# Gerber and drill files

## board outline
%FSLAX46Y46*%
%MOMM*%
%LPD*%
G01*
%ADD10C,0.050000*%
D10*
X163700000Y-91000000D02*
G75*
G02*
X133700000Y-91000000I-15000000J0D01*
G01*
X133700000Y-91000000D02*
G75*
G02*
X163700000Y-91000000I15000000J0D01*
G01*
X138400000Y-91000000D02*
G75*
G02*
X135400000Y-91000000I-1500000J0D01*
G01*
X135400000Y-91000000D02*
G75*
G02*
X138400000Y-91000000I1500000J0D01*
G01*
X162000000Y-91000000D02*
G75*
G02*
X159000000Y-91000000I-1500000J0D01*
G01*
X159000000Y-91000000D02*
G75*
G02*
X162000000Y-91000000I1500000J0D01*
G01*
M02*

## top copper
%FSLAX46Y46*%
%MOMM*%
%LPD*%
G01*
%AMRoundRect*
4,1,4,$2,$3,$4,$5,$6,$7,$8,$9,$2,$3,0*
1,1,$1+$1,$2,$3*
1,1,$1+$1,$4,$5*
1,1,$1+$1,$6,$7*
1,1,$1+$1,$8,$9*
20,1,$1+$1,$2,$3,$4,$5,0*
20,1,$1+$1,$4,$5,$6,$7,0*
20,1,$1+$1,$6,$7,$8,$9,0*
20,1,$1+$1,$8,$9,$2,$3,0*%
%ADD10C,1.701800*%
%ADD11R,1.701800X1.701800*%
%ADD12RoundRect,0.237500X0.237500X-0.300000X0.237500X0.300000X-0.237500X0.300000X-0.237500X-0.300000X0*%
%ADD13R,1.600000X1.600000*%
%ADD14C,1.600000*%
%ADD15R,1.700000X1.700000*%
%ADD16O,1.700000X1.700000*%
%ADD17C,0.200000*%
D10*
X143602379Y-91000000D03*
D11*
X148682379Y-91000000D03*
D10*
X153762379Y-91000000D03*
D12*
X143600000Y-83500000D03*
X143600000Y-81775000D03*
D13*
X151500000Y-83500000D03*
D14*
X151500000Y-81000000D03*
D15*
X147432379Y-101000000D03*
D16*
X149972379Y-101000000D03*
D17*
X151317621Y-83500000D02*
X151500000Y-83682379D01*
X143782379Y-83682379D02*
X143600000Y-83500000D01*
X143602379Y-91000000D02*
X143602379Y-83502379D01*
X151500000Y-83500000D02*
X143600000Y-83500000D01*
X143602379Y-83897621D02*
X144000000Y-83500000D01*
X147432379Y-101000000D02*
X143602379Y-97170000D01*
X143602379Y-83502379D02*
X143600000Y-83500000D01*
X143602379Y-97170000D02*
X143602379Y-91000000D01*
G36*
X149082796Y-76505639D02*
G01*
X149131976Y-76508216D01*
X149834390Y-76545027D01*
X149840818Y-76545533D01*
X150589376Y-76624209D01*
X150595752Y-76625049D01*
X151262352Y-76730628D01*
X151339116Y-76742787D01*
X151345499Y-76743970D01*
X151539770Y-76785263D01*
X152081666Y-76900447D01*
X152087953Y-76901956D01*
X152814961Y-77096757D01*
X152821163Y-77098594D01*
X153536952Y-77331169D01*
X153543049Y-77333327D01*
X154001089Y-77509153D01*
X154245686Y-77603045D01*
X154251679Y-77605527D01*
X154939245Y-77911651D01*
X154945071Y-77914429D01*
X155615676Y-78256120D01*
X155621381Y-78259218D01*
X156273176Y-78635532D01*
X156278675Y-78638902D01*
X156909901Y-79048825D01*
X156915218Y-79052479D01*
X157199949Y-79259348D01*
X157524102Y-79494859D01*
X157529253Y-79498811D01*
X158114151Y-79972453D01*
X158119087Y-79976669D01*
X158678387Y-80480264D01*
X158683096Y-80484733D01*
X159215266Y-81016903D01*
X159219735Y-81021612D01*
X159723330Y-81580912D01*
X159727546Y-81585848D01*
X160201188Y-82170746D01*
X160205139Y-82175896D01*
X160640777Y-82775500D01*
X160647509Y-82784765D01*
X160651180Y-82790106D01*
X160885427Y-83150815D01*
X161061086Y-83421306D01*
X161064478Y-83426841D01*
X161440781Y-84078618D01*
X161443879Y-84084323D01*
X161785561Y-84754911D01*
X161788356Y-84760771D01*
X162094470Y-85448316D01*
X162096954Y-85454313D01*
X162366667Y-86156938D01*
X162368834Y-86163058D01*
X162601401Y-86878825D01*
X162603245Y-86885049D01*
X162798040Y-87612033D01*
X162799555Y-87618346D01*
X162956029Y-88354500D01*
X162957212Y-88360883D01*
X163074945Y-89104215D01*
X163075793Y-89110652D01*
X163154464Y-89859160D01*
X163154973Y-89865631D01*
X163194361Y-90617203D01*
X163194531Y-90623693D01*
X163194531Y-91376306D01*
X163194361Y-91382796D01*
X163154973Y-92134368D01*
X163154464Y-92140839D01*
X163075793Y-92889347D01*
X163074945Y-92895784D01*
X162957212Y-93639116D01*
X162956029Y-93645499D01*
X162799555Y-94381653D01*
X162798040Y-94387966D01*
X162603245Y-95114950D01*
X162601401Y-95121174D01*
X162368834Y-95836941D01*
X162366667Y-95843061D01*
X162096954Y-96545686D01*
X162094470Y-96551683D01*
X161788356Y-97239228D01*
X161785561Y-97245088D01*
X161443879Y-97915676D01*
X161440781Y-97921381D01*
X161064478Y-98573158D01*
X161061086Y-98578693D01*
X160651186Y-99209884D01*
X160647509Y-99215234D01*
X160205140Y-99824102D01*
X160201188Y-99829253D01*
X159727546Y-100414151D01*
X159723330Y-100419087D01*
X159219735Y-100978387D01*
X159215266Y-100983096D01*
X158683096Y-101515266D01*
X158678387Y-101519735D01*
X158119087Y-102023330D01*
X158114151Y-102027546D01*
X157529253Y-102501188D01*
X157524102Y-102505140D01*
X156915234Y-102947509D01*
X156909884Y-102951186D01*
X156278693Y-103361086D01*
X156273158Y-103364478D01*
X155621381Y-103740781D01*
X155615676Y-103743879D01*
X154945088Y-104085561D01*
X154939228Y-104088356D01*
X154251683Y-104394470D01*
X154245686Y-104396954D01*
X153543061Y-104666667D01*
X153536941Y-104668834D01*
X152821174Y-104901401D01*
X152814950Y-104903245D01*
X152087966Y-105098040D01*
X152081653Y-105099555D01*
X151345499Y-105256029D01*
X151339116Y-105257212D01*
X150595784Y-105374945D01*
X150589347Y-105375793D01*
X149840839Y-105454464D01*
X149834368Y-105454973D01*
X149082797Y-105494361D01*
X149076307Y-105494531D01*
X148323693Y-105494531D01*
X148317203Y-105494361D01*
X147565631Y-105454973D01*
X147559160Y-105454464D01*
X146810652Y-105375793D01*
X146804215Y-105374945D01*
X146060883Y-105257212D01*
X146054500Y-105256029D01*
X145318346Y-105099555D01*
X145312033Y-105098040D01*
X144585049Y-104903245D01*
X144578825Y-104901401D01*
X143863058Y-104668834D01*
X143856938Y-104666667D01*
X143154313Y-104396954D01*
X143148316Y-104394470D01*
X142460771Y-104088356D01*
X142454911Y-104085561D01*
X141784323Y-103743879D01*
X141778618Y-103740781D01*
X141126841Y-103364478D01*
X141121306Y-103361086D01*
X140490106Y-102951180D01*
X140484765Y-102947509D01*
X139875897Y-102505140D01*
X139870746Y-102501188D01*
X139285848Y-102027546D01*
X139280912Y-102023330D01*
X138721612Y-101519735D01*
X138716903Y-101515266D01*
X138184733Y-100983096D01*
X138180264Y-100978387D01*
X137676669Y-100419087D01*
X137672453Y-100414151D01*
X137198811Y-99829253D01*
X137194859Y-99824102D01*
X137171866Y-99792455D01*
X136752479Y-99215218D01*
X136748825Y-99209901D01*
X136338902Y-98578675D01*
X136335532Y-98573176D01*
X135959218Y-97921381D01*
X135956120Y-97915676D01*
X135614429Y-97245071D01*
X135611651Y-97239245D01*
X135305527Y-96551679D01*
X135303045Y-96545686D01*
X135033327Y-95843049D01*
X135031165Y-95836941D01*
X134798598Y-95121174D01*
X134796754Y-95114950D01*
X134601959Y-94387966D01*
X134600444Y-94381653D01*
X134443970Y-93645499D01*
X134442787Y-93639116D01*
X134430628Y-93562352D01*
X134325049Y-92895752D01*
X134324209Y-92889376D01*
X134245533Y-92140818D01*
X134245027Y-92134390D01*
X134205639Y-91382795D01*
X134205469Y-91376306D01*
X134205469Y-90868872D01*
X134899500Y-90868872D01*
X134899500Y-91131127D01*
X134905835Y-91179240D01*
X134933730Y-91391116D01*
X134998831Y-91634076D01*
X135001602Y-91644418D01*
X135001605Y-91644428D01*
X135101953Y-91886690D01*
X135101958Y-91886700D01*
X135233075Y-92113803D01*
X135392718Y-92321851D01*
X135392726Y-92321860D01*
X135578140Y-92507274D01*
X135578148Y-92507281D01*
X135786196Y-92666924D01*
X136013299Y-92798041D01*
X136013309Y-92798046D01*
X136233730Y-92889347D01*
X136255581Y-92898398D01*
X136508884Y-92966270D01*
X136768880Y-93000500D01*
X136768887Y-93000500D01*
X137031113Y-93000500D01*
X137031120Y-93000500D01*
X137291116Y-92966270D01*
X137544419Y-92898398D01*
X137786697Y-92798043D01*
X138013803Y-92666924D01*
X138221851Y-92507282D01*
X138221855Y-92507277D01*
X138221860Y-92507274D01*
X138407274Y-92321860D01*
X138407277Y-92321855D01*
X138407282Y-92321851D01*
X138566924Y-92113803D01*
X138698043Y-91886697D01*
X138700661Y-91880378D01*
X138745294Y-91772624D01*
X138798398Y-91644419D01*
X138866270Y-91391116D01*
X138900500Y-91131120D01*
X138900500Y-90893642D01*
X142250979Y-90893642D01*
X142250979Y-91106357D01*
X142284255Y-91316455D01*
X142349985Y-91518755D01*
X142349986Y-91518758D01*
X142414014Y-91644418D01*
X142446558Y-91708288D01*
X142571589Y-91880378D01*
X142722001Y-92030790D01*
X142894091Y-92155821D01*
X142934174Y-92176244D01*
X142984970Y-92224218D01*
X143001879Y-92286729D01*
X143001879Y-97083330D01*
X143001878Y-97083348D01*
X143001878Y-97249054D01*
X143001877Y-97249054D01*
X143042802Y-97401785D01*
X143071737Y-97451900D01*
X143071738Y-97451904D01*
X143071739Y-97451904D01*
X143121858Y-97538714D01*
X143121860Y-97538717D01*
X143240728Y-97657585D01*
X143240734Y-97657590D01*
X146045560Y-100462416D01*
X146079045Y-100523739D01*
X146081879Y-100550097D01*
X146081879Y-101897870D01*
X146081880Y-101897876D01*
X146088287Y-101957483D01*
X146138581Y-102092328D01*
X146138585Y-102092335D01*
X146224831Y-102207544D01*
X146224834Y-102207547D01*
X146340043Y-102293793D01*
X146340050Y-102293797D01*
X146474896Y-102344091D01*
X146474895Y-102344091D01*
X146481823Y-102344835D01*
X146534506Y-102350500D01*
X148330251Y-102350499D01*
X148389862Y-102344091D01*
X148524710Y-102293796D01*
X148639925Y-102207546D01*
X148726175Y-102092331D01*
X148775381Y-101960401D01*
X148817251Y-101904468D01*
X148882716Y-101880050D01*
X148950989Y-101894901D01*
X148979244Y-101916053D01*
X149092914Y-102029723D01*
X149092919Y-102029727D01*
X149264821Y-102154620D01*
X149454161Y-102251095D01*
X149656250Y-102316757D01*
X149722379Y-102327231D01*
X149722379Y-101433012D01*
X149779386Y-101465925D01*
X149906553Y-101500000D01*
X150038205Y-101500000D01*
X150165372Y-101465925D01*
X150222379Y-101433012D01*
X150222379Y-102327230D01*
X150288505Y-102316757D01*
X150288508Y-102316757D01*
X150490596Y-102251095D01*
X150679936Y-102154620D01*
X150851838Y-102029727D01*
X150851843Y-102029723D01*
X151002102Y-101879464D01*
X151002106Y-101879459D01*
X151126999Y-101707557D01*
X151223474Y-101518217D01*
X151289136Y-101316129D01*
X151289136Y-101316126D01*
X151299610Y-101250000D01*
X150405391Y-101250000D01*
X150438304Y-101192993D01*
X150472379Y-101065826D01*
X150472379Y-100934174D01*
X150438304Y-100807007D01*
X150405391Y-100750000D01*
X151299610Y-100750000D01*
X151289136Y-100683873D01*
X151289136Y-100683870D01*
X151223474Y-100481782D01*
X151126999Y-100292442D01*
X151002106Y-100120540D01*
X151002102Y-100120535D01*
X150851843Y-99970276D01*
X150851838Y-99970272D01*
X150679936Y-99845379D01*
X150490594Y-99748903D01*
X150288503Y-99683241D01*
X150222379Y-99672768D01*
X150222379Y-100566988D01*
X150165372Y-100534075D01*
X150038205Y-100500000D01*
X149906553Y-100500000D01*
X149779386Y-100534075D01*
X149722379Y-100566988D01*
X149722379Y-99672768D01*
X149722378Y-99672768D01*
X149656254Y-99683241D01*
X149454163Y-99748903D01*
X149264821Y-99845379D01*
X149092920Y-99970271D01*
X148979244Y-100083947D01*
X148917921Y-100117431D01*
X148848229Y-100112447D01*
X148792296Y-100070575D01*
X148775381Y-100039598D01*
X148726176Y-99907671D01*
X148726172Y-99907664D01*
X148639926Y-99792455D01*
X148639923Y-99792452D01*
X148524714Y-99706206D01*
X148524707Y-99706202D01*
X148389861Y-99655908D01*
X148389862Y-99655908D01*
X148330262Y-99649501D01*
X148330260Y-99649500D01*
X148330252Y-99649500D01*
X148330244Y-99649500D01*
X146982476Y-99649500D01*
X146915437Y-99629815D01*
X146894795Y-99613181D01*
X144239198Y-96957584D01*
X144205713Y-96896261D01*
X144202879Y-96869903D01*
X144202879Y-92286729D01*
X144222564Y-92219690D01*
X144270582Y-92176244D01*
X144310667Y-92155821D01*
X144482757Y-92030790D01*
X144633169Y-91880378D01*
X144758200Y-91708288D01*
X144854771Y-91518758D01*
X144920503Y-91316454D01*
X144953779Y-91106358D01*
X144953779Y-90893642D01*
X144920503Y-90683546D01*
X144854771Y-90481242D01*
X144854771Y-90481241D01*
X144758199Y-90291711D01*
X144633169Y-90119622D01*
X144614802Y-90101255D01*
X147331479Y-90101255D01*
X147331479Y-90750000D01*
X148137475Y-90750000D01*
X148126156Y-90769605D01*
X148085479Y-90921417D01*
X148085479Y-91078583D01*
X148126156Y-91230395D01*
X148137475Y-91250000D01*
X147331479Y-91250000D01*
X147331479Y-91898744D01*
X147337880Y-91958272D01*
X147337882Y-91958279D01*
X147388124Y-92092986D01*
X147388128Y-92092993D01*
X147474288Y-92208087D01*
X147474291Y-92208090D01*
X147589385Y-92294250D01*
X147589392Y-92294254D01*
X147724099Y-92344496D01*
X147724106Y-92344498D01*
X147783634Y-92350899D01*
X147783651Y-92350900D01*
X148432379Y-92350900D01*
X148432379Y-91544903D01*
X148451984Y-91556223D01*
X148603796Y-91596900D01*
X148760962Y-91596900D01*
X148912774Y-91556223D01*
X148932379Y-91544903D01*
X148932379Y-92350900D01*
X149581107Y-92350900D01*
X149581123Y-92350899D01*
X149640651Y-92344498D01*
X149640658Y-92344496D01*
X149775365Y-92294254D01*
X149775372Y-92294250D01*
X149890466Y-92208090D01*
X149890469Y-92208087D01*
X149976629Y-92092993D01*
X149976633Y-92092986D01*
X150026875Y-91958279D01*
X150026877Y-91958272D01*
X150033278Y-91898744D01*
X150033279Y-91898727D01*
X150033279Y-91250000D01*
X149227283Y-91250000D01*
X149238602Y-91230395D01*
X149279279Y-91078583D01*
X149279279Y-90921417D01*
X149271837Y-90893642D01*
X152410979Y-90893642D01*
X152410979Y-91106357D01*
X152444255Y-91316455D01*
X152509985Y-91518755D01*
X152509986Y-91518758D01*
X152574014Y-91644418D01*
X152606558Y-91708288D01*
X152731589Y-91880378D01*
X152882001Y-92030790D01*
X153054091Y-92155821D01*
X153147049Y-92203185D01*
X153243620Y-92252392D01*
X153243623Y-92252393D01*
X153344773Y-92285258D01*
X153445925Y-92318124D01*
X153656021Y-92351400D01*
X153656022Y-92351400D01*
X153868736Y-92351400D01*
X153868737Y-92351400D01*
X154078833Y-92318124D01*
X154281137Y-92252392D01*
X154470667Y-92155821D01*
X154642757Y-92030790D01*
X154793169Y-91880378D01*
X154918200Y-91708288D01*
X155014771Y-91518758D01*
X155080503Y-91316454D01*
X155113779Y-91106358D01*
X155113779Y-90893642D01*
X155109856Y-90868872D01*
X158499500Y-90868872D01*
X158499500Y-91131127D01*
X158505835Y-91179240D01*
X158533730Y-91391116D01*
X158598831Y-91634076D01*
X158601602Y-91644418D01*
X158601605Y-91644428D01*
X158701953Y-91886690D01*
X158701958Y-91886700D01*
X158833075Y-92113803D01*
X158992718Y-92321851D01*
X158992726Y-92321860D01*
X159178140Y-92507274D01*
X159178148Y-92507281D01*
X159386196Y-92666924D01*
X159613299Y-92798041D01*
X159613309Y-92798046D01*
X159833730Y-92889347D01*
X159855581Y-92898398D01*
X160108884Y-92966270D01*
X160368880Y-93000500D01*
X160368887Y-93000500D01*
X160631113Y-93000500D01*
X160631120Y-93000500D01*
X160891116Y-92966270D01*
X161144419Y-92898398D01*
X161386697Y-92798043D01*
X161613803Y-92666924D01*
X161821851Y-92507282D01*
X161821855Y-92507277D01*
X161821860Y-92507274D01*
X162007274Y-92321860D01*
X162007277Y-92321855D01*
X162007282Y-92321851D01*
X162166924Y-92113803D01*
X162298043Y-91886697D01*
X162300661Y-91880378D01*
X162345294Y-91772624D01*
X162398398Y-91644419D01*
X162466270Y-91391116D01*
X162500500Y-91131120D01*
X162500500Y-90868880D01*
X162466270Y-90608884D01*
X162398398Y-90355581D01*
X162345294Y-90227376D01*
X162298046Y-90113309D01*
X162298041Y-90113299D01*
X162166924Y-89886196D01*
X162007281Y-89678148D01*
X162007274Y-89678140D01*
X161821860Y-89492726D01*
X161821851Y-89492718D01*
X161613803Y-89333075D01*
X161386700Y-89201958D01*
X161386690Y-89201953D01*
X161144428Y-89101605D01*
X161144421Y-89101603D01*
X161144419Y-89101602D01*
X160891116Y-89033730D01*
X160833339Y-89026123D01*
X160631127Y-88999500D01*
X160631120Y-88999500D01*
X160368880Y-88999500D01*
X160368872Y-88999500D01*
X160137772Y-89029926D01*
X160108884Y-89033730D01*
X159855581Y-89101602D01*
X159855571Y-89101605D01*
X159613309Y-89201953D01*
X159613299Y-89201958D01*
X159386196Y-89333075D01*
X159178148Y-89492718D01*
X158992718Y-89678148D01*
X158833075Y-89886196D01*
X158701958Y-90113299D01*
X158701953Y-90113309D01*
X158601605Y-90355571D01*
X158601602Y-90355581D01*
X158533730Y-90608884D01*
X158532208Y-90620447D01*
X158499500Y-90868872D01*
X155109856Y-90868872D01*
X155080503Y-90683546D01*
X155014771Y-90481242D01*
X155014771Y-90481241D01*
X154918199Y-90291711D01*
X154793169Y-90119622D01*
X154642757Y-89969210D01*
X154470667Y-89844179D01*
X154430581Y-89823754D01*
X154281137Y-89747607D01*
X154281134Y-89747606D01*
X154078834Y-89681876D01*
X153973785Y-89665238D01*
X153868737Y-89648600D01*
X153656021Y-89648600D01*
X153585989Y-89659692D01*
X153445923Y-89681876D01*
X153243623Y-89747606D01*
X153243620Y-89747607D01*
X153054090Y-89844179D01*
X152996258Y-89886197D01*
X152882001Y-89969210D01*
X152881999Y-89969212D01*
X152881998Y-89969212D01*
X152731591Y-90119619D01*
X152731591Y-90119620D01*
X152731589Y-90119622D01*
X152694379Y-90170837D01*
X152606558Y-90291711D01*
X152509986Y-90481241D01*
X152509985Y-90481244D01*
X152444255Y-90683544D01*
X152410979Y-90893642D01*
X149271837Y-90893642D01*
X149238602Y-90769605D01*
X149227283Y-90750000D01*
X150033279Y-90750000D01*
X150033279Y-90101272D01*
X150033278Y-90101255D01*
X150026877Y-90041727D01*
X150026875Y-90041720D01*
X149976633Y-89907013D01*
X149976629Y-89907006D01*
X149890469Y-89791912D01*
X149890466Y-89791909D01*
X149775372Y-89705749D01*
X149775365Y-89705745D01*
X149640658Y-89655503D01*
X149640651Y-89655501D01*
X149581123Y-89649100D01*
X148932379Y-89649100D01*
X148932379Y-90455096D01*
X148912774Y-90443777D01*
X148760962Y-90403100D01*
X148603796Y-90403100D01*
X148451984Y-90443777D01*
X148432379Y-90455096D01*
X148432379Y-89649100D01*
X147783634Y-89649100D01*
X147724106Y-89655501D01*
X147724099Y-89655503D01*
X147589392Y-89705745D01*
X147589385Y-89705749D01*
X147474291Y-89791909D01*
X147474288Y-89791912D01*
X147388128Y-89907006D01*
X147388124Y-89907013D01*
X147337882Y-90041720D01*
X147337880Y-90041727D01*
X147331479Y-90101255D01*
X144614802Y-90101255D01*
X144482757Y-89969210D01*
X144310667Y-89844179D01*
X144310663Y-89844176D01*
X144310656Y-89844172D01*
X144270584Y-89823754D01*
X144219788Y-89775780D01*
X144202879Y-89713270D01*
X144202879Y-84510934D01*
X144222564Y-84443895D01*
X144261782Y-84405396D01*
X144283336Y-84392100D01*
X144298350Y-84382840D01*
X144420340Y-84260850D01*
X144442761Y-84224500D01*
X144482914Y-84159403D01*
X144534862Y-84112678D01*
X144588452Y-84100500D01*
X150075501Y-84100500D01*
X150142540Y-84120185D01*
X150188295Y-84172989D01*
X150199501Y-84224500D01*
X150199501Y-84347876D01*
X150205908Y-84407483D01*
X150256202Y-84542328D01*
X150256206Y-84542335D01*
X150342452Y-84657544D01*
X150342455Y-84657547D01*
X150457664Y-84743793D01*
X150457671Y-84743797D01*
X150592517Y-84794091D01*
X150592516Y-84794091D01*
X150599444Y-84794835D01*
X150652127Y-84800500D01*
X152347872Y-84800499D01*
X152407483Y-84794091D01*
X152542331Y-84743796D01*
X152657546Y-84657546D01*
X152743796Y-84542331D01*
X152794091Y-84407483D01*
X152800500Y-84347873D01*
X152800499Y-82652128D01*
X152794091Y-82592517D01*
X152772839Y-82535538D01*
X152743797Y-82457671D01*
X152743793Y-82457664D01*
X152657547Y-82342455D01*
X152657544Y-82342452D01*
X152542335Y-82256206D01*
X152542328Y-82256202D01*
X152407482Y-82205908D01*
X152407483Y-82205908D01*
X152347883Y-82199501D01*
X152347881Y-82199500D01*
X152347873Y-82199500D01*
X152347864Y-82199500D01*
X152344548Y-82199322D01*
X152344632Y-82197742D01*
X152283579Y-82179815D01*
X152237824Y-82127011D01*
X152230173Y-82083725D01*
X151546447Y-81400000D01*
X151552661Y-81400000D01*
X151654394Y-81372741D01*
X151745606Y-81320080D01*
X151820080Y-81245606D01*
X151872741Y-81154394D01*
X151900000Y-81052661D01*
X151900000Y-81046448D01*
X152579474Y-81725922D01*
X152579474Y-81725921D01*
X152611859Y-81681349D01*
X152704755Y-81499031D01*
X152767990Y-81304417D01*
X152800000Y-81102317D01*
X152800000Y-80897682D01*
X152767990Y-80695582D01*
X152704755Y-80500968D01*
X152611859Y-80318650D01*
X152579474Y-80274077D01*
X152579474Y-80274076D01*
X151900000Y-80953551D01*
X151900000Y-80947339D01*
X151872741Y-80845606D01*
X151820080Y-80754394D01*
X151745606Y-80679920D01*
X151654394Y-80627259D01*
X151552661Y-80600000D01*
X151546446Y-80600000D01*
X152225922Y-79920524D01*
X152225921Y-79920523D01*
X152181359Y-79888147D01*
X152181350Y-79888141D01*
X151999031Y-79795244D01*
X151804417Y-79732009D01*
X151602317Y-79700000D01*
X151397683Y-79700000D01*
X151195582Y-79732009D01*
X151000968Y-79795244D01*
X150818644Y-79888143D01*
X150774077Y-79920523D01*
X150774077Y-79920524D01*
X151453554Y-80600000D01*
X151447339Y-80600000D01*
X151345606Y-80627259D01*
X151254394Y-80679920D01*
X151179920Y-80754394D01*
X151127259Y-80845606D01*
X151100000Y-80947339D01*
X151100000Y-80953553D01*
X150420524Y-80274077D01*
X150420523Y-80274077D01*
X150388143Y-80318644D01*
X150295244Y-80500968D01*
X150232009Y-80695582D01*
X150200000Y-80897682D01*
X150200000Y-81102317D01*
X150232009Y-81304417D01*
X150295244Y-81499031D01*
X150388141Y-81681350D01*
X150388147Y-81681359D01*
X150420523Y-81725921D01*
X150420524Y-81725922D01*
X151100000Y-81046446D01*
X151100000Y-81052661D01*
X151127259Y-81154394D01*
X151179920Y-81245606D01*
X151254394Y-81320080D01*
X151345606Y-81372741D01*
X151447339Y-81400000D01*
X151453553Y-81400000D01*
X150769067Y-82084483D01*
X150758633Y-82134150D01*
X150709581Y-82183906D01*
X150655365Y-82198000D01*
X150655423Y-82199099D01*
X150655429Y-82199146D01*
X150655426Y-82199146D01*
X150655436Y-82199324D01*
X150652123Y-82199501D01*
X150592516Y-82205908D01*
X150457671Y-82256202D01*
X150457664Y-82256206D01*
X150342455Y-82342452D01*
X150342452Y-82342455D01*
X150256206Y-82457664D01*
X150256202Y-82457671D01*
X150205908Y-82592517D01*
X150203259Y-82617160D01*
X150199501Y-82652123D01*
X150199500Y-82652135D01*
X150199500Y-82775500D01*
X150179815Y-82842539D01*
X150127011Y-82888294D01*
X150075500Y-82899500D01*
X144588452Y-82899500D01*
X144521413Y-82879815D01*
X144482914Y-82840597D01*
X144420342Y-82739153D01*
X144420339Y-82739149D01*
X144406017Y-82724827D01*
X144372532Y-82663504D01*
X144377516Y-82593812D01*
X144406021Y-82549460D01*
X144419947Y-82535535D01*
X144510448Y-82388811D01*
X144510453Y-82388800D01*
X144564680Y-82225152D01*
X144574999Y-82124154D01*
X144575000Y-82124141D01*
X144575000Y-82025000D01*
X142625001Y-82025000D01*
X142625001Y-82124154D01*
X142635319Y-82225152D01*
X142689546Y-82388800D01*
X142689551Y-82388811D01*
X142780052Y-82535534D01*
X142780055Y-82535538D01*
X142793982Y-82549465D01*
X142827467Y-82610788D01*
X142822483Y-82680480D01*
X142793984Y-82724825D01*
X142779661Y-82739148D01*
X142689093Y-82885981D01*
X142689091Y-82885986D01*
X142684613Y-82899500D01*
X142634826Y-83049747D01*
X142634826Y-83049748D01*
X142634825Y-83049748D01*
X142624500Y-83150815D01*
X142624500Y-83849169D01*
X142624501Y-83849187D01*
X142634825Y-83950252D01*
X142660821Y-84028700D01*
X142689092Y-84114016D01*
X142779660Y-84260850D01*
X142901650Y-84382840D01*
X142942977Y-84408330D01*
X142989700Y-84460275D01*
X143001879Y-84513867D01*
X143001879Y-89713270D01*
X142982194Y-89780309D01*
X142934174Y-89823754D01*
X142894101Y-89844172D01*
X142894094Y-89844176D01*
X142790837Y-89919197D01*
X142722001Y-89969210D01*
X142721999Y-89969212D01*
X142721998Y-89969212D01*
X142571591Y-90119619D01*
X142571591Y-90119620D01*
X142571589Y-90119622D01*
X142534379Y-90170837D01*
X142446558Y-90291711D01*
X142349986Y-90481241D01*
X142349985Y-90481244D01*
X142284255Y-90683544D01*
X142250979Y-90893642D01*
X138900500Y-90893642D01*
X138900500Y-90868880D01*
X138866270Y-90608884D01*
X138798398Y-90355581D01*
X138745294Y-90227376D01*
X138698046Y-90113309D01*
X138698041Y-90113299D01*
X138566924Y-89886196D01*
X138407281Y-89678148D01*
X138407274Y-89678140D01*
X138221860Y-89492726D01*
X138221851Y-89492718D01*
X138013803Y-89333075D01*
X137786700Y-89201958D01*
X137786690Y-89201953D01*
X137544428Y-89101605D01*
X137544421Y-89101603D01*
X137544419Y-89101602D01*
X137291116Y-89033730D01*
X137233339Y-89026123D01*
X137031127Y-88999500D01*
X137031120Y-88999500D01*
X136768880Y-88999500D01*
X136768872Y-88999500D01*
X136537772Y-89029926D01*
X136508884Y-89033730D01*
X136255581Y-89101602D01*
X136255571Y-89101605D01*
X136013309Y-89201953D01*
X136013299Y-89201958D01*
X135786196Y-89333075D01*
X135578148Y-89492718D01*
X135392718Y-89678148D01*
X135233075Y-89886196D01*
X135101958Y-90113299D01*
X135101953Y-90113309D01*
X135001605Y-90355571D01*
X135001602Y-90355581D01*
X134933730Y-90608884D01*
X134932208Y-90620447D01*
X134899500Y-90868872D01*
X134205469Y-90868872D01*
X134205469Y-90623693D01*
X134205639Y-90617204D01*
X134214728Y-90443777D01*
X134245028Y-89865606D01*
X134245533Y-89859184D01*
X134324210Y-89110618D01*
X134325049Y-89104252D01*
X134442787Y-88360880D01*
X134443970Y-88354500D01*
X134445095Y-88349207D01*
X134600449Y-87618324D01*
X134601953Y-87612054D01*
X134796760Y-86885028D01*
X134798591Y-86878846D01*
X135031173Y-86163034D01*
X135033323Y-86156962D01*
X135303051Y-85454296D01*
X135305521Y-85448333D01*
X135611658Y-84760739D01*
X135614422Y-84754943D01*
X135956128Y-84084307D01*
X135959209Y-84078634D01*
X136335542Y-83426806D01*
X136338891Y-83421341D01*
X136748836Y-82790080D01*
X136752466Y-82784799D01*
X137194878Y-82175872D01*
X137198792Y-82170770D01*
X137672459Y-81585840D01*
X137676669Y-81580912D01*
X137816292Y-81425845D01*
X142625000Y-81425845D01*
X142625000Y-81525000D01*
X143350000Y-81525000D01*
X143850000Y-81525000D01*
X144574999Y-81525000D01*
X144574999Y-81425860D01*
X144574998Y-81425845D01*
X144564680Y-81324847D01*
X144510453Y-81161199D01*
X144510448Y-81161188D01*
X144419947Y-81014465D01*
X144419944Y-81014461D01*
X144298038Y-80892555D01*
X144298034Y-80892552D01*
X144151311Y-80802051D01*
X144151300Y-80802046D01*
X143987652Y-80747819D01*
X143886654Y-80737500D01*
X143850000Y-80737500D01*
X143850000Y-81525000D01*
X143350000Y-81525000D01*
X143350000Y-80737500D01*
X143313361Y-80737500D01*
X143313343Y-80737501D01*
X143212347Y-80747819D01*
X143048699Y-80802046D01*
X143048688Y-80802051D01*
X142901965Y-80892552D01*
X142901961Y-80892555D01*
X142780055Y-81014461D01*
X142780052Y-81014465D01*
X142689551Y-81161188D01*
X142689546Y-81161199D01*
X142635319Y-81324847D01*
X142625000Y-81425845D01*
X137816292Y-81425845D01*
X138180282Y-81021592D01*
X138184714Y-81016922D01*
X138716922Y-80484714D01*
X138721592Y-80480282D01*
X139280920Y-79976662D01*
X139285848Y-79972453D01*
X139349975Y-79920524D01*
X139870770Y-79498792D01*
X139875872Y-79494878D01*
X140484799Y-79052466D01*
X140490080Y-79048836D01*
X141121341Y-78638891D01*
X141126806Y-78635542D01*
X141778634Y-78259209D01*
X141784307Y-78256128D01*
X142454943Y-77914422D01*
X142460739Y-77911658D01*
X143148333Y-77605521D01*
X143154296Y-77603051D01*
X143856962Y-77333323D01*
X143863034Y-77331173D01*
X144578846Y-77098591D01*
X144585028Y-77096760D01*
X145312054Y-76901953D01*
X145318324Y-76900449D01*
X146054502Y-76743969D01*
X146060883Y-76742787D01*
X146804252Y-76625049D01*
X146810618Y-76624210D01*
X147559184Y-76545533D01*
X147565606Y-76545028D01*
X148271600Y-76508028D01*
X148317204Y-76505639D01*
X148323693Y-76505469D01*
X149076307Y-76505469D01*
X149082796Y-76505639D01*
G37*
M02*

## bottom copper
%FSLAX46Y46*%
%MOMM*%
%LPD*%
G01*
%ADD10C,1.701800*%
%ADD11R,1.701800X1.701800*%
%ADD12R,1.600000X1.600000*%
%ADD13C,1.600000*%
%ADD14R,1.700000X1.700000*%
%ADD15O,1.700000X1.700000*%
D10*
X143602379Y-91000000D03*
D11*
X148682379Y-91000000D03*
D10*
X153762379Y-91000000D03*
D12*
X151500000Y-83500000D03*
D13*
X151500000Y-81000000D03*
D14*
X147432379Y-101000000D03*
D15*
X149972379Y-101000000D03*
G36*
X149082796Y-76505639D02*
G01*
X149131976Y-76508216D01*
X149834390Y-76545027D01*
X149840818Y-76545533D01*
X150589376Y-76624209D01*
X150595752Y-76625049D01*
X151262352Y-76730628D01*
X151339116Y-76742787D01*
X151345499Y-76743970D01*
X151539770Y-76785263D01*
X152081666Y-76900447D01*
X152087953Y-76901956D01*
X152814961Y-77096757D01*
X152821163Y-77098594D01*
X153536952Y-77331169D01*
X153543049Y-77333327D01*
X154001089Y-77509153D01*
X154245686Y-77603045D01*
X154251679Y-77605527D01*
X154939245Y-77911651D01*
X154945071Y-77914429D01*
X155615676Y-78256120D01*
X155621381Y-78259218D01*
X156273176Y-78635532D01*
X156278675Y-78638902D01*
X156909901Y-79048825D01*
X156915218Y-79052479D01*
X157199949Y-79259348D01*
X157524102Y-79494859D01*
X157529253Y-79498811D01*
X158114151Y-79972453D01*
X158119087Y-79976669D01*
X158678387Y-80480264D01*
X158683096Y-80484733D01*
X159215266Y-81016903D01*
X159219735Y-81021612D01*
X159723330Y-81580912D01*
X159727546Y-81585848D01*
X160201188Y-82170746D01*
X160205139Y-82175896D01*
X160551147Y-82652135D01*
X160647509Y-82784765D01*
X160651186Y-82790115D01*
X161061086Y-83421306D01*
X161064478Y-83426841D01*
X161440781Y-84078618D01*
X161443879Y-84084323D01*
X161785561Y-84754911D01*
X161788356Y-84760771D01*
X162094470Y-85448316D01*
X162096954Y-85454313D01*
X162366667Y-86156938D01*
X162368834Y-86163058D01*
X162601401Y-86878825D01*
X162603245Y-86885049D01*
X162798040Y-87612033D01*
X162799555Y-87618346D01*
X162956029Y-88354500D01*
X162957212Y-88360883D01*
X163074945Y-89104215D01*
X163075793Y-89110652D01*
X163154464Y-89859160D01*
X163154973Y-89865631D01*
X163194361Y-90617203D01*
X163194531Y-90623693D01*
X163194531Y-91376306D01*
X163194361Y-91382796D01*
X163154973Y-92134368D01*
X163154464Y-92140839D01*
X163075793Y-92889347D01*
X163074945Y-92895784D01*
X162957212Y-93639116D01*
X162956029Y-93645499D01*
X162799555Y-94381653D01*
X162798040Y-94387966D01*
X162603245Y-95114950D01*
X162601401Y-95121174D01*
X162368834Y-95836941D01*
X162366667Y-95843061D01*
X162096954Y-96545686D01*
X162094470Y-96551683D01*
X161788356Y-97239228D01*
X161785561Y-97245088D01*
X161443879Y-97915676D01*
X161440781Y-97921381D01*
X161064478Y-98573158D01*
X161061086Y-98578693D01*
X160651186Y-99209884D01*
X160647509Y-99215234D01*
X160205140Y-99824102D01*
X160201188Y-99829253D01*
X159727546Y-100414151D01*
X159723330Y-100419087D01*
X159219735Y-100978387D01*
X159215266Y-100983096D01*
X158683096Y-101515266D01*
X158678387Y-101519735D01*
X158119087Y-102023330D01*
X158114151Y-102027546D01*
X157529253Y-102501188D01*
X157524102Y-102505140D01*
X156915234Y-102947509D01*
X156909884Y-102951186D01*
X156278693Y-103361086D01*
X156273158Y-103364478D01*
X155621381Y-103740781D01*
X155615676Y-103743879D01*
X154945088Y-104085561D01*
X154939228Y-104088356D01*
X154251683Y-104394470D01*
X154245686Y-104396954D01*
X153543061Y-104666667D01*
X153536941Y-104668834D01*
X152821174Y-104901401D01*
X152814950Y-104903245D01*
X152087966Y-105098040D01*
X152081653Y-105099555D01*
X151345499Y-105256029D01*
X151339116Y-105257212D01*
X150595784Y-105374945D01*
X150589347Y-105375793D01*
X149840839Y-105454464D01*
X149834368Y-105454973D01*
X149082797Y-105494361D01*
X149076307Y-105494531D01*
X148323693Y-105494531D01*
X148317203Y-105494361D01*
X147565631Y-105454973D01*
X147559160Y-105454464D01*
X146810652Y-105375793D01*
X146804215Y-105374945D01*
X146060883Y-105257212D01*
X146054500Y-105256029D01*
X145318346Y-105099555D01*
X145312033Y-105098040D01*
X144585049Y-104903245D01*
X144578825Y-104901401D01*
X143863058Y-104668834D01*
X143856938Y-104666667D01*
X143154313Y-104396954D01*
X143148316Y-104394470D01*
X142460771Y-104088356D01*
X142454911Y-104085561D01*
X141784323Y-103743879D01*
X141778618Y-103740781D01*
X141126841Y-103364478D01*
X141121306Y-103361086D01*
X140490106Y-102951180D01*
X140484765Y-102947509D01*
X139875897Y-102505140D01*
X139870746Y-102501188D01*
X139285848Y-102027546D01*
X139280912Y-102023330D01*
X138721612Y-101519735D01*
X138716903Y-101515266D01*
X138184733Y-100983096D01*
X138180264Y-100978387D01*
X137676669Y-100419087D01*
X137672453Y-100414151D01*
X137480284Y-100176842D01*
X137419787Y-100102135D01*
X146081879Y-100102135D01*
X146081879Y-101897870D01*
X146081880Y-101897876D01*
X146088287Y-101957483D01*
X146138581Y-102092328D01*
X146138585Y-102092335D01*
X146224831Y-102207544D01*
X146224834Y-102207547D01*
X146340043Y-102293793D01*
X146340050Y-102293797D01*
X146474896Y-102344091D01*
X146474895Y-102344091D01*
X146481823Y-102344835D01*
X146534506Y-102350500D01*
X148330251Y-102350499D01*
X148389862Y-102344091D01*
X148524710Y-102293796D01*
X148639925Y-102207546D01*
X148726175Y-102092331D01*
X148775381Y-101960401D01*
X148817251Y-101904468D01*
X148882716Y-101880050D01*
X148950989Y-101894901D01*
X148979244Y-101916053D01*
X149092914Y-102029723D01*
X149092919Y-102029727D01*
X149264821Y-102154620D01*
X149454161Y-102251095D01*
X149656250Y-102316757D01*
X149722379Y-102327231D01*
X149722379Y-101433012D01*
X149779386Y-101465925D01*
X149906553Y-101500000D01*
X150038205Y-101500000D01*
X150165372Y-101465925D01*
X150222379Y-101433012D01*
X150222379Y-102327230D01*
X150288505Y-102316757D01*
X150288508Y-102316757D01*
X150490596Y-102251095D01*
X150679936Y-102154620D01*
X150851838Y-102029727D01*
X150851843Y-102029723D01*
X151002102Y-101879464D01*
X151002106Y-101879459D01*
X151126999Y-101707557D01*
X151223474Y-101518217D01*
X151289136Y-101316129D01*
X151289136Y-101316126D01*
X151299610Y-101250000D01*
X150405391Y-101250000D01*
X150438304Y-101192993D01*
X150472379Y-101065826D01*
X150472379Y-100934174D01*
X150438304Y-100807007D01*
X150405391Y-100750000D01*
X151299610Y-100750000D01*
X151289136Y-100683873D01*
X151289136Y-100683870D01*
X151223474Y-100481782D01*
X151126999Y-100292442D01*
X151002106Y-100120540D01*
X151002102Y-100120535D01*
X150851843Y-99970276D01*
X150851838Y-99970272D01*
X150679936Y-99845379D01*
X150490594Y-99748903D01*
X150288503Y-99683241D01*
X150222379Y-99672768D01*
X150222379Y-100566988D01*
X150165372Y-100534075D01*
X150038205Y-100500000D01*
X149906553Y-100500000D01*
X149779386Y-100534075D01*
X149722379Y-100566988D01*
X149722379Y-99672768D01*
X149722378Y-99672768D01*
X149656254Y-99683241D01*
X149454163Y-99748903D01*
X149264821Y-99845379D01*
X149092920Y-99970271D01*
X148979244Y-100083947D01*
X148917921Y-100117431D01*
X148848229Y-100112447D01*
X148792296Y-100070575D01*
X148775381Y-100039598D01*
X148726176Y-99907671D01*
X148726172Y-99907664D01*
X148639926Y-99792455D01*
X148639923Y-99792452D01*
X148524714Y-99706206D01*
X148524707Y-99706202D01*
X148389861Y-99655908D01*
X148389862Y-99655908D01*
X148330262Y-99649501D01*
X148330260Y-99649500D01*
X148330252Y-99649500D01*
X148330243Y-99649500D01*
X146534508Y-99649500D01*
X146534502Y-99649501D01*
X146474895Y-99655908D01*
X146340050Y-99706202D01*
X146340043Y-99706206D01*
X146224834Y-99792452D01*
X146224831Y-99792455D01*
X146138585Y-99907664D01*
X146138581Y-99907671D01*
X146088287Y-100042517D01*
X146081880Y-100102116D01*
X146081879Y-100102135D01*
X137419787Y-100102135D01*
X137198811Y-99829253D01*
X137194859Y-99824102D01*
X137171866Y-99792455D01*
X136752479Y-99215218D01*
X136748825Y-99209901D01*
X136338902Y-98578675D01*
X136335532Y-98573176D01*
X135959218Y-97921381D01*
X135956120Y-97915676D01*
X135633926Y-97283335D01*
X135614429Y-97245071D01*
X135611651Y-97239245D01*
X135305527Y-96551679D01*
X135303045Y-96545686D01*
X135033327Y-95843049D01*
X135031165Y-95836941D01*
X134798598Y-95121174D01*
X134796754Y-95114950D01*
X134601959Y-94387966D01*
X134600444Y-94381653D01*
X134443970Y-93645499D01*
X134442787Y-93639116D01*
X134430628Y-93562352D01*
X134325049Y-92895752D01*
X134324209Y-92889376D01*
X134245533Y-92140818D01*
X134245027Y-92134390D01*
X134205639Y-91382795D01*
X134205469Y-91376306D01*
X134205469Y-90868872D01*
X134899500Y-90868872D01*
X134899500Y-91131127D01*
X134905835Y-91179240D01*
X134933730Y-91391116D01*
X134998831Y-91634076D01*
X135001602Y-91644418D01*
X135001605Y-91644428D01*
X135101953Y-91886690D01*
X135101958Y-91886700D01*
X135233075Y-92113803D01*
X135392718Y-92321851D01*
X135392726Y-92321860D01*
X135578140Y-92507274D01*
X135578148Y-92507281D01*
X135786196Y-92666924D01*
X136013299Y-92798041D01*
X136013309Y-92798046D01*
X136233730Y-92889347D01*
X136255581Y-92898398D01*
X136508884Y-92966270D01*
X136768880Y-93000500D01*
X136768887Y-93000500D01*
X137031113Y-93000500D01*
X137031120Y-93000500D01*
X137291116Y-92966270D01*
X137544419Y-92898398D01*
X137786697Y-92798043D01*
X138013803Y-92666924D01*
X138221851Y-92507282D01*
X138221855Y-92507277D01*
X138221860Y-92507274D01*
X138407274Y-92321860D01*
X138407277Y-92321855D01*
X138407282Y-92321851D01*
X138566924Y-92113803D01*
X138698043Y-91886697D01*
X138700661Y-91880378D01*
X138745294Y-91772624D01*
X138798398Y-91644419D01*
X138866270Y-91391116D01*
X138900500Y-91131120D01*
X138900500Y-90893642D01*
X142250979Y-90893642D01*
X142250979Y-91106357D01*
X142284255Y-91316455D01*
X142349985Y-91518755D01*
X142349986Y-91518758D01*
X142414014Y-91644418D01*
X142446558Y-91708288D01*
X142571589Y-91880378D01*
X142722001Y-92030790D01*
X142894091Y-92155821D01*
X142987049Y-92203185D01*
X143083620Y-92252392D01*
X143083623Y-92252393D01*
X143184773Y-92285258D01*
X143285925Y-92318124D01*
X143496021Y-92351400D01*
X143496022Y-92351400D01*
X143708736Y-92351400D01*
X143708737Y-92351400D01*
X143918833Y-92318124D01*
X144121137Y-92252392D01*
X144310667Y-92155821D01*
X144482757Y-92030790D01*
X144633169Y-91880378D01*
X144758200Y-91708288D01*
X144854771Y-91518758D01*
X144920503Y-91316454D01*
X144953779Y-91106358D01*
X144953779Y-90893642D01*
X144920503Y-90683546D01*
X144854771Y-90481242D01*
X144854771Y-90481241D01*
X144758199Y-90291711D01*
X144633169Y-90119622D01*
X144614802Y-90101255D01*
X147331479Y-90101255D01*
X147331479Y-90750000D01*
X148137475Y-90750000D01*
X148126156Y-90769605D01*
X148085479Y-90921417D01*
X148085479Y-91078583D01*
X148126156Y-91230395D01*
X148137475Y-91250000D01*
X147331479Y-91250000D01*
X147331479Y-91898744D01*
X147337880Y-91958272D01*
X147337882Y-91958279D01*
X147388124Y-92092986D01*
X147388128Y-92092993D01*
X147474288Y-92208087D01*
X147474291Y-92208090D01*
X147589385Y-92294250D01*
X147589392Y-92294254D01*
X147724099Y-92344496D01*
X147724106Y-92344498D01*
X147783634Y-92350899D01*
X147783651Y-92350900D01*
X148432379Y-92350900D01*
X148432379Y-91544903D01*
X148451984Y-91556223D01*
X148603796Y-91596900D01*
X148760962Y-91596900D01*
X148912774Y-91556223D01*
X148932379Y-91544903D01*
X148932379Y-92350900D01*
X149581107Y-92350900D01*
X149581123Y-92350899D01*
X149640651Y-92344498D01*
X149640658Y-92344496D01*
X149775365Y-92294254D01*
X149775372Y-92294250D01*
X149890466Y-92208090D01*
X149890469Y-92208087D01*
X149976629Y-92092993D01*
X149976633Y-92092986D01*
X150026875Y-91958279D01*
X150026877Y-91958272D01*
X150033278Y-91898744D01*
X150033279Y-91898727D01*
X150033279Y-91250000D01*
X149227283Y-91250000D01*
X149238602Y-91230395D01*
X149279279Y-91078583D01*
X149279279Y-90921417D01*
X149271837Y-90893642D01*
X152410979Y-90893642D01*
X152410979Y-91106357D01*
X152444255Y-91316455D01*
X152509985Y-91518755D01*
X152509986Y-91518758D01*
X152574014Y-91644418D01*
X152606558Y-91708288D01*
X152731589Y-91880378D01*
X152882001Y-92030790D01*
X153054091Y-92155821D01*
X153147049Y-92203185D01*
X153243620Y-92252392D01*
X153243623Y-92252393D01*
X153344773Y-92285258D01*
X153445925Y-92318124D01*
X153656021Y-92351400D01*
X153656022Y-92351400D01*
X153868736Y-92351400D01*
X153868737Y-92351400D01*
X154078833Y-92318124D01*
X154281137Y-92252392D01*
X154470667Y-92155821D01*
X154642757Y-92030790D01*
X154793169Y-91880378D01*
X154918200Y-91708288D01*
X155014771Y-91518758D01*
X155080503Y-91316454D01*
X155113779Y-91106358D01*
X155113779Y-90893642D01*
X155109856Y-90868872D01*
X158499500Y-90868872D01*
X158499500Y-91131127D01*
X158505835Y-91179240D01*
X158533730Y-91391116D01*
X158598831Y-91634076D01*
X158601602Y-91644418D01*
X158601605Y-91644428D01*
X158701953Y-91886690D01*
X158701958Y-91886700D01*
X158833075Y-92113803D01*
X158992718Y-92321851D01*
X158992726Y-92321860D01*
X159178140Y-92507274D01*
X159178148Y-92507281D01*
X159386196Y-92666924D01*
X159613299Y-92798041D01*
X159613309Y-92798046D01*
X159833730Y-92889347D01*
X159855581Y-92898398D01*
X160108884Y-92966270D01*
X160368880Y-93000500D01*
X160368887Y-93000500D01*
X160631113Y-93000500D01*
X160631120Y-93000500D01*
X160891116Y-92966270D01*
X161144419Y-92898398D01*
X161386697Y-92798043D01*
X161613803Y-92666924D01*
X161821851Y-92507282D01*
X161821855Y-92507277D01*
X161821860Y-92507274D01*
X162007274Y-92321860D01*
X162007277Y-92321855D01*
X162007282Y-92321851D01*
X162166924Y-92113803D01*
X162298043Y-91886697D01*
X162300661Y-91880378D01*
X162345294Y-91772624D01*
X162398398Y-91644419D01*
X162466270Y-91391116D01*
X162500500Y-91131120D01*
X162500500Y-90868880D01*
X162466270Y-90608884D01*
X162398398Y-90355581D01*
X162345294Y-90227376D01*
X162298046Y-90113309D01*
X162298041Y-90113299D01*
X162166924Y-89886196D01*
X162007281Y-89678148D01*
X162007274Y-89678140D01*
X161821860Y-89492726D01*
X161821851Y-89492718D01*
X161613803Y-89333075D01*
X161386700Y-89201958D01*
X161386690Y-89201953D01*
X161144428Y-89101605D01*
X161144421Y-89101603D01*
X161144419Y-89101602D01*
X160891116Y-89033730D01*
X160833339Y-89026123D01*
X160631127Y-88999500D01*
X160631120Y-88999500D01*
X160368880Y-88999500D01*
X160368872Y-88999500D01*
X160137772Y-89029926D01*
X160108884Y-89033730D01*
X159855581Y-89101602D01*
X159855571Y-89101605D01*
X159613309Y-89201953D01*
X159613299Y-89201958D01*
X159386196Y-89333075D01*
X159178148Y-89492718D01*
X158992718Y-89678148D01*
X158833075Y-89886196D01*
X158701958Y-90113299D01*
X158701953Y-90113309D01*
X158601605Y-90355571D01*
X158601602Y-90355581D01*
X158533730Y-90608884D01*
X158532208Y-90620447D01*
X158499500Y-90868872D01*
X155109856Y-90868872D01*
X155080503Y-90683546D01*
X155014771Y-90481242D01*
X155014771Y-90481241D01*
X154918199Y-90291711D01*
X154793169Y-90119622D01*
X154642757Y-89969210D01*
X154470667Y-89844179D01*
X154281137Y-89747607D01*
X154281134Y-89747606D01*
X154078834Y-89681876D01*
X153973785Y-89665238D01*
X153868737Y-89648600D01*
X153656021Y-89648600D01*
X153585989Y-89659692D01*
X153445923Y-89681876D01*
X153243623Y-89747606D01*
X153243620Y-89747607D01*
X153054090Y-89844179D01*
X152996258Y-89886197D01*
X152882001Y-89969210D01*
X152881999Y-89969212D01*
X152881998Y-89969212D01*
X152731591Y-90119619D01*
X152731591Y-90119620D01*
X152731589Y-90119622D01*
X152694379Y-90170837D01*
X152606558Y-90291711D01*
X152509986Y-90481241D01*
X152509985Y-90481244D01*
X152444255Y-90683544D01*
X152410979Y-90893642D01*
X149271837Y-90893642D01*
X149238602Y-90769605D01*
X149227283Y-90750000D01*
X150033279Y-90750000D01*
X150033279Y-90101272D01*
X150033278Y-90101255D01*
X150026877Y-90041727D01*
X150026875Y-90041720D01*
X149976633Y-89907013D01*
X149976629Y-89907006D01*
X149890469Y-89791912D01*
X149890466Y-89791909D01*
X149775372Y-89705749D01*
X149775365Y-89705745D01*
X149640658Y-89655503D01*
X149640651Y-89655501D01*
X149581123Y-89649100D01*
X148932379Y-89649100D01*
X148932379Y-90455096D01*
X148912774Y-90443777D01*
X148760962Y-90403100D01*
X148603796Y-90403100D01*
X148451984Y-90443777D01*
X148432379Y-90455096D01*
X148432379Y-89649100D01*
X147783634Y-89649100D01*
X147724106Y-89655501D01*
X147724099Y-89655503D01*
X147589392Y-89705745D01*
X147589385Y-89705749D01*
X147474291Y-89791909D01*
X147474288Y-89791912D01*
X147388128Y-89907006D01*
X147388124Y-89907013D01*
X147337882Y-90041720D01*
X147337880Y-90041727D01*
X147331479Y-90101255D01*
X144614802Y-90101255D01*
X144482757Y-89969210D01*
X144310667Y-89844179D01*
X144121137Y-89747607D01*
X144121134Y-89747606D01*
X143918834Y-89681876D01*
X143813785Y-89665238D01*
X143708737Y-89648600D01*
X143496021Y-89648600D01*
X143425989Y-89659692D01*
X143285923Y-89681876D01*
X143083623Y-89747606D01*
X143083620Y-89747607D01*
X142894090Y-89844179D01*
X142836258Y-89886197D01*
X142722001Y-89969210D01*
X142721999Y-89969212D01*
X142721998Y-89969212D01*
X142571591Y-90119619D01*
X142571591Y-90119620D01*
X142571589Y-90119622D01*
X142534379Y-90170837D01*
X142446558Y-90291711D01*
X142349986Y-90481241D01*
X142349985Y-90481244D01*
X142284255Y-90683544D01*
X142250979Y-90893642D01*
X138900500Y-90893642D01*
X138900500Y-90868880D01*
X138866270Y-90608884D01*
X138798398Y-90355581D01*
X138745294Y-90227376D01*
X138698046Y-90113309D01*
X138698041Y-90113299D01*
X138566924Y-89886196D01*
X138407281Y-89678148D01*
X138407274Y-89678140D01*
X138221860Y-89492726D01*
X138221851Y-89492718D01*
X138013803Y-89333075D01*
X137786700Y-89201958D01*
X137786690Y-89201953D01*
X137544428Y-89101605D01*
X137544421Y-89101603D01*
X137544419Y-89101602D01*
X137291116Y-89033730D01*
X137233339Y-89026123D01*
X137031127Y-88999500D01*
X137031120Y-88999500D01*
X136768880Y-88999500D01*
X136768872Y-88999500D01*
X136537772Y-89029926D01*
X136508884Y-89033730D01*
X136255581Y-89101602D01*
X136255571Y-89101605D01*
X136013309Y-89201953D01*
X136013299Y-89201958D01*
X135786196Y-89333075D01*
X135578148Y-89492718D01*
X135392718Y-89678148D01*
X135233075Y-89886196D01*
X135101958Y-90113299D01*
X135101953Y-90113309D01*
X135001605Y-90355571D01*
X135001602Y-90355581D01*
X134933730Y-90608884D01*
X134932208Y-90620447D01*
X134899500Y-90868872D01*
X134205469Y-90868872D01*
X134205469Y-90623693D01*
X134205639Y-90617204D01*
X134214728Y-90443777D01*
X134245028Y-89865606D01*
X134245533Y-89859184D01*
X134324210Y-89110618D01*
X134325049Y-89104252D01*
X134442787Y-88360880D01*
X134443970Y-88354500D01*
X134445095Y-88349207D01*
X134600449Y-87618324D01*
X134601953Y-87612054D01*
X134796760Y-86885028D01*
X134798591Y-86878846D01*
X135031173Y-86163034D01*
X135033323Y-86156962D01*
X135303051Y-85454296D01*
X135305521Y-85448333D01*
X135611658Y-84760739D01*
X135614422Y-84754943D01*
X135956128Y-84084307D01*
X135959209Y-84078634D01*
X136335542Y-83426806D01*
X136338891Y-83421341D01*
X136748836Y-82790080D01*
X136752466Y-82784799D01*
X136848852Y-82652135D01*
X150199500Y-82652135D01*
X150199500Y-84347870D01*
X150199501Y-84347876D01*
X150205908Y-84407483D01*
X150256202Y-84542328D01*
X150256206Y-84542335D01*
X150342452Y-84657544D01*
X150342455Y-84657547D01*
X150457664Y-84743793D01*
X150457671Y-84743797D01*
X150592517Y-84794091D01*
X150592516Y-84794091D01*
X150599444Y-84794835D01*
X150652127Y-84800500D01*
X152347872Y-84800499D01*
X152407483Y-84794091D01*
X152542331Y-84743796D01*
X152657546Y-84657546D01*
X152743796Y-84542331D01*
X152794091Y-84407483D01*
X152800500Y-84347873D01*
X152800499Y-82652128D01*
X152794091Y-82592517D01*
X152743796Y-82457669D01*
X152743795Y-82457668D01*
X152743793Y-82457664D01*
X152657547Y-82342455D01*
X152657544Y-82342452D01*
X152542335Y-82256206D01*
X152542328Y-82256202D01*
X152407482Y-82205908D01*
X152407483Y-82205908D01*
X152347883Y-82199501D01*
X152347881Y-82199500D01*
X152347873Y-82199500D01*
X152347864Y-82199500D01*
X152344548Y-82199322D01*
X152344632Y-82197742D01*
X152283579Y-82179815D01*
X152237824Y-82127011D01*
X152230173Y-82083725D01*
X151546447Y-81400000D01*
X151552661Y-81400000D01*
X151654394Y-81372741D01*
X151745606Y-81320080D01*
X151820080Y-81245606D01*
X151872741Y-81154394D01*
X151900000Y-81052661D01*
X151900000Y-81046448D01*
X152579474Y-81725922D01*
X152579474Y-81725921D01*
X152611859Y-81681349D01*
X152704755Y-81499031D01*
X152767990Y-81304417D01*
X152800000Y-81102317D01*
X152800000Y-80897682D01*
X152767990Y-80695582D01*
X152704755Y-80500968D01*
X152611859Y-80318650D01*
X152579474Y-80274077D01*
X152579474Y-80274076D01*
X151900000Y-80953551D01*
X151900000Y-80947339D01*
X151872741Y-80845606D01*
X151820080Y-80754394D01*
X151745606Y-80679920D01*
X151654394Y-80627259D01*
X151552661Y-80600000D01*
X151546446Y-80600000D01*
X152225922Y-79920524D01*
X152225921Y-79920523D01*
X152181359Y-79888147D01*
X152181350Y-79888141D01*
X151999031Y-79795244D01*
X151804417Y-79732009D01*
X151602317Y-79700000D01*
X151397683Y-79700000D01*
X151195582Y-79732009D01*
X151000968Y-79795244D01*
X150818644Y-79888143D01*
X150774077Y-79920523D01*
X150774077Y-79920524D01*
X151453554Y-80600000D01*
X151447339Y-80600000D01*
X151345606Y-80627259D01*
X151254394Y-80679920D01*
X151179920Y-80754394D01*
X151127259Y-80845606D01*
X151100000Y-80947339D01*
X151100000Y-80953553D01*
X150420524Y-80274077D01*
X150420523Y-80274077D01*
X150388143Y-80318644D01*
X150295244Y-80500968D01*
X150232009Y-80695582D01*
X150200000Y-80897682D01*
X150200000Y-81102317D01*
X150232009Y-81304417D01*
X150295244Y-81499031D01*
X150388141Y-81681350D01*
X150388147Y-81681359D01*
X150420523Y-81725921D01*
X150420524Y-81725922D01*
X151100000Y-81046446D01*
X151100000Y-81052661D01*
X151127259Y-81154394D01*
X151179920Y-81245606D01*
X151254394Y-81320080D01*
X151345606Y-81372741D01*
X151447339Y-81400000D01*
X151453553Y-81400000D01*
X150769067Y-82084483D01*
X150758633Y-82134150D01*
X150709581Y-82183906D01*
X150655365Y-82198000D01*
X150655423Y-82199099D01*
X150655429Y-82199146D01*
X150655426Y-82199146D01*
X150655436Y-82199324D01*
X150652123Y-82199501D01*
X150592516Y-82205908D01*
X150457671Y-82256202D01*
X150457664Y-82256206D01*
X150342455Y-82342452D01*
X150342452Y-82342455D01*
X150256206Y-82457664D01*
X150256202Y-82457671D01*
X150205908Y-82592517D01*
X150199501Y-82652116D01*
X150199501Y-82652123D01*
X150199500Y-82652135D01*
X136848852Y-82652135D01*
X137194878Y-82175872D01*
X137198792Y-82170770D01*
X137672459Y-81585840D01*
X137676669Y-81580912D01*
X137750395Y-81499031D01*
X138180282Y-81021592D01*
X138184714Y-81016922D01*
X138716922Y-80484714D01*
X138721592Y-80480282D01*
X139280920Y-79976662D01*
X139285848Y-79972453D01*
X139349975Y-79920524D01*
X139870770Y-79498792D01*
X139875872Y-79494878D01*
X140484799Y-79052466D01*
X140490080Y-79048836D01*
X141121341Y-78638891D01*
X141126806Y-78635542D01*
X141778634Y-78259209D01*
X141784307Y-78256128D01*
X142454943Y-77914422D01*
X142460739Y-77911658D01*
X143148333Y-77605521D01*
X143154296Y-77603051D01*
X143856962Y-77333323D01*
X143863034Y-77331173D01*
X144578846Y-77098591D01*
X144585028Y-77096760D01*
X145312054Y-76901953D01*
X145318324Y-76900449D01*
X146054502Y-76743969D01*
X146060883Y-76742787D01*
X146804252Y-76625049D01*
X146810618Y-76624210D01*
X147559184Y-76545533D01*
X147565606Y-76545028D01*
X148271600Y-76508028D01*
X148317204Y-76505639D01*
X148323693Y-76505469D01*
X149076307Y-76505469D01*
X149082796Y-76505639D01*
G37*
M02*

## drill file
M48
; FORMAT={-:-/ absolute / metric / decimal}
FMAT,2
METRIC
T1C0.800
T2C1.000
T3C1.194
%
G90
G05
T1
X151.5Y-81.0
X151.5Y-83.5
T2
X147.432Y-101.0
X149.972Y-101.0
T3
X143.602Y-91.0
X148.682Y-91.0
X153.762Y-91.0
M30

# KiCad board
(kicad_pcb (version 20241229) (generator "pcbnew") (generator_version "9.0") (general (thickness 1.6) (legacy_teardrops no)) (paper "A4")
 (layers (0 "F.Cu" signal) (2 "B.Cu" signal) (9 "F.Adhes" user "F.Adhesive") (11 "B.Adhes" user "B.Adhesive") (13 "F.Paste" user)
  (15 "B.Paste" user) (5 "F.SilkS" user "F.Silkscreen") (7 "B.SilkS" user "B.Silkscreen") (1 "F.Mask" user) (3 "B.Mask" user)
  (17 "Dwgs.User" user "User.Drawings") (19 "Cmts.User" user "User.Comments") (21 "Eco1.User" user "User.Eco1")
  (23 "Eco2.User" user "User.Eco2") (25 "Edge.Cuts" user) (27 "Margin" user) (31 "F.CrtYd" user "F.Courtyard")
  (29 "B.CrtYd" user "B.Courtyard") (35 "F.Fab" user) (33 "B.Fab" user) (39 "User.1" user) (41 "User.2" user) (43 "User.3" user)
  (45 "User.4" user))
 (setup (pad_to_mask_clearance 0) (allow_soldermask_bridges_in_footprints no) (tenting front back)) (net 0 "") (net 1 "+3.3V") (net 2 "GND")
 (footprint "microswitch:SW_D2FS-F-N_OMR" (layer "F.Cu") (at 143.602379 91)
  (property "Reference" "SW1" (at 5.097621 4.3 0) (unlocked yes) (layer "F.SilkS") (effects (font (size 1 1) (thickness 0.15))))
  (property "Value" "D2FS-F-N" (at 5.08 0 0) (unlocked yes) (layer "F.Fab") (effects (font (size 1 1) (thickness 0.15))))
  (pad "1" thru_hole circle (at 0 0) (size 1.7018 1.7018) (drill 1.1938) (layers "*.Cu" "*.Mask") (remove_unused_layers no) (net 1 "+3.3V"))
  (pad "2" thru_hole rect (at 5.08 0) (size 1.7018 1.7018) (drill 1.1938) (layers "*.Cu" "*.Mask") (remove_unused_layers no) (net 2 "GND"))
  (pad "3" thru_hole circle (at 10.16 0) (size 1.7018 1.7018) (drill 1.1938) (layers "*.Cu" "*.Mask") (remove_unused_layers no)))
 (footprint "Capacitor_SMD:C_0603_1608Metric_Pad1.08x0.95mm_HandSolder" (layer "F.Cu") (at 143.6 82.6375 90)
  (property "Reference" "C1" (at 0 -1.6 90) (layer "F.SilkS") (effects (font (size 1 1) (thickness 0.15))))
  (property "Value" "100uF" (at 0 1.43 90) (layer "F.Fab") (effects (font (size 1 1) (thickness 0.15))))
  (pad "1" smd roundrect (at -0.8625 0 90) (size 1.075 0.95) (layers "F.Cu" "F.Mask" "F.Paste") (roundrect_rratio 0.25) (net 1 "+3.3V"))
  (pad "2" smd roundrect (at 0.8625 0 90) (size 1.075 0.95) (layers "F.Cu" "F.Mask" "F.Paste") (roundrect_rratio 0.25) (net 2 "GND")))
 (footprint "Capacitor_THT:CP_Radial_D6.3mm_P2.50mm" (layer "F.Cu") (at 151.5 83.5 90)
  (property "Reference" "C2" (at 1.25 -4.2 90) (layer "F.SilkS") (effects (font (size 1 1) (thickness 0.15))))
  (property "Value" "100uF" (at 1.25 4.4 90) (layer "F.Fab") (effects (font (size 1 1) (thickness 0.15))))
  (pad "1" thru_hole rect (at 0 0 90) (size 1.6 1.6) (drill 0.8) (layers "*.Cu" "*.Mask") (remove_unused_layers no) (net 1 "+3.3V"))
  (pad "2" thru_hole circle (at 2.5 0 90) (size 1.6 1.6) (drill 0.8) (layers "*.Cu" "*.Mask") (remove_unused_layers no) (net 2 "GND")))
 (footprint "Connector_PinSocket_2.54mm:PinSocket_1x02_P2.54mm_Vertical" (layer "F.Cu") (at 147.432379 101 90)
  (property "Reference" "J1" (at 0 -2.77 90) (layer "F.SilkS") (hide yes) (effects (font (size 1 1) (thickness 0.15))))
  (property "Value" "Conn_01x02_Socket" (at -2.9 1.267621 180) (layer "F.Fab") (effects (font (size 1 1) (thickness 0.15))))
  (pad "1" thru_hole rect (at 0 0 90) (size 1.7 1.7) (drill 1) (layers "*.Cu" "*.Mask") (remove_unused_layers no) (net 1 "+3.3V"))
  (pad "2" thru_hole oval (at 0 2.54 90) (size 1.7 1.7) (drill 1) (layers "*.Cu" "*.Mask") (remove_unused_layers no) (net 2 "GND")))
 (gr_circle (center 148.7 91) (end 163.7 91) (stroke (width 0.05) (type solid)) (fill no) (layer "Edge.Cuts"))
 (gr_circle (center 136.9 91) (end 138.4 91) (stroke (width 0.05) (type solid)) (fill no) (layer "Edge.Cuts"))
 (gr_circle (center 160.5 91) (end 162 91) (stroke (width 0.05) (type solid)) (fill no) (layer "Edge.Cuts"))
 (segment (start 151.317621 83.5) (end 151.5 83.682379) (width 0.2) (layer "F.Cu") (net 1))
 (segment (start 143.782379 83.682379) (end 143.6 83.5) (width 0.2) (layer "F.Cu") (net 1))
 (segment (start 143.602379 91) (end 143.602379 83.502379) (width 0.2) (layer "F.Cu") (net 1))
 (segment (start 151.5 83.5) (end 143.6 83.5) (width 0.2) (layer "F.Cu") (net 1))
 (segment (start 143.602379 83.897621) (end 144 83.5) (width 0.2) (layer "F.Cu") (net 1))
 (segment (start 147.432379 101) (end 143.602379 97.17) (width 0.2) (layer "F.Cu") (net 1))
 (segment (start 143.602379 83.502379) (end 143.6 83.5) (width 0.2) (layer "F.Cu") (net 1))
 (segment (start 143.602379 97.17) (end 143.602379 91) (width 0.2) (layer "F.Cu") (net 1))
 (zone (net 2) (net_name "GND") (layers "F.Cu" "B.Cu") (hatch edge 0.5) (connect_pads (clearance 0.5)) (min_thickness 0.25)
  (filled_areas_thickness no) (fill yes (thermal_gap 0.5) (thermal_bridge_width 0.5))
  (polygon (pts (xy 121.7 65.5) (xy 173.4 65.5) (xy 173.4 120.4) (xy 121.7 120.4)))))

